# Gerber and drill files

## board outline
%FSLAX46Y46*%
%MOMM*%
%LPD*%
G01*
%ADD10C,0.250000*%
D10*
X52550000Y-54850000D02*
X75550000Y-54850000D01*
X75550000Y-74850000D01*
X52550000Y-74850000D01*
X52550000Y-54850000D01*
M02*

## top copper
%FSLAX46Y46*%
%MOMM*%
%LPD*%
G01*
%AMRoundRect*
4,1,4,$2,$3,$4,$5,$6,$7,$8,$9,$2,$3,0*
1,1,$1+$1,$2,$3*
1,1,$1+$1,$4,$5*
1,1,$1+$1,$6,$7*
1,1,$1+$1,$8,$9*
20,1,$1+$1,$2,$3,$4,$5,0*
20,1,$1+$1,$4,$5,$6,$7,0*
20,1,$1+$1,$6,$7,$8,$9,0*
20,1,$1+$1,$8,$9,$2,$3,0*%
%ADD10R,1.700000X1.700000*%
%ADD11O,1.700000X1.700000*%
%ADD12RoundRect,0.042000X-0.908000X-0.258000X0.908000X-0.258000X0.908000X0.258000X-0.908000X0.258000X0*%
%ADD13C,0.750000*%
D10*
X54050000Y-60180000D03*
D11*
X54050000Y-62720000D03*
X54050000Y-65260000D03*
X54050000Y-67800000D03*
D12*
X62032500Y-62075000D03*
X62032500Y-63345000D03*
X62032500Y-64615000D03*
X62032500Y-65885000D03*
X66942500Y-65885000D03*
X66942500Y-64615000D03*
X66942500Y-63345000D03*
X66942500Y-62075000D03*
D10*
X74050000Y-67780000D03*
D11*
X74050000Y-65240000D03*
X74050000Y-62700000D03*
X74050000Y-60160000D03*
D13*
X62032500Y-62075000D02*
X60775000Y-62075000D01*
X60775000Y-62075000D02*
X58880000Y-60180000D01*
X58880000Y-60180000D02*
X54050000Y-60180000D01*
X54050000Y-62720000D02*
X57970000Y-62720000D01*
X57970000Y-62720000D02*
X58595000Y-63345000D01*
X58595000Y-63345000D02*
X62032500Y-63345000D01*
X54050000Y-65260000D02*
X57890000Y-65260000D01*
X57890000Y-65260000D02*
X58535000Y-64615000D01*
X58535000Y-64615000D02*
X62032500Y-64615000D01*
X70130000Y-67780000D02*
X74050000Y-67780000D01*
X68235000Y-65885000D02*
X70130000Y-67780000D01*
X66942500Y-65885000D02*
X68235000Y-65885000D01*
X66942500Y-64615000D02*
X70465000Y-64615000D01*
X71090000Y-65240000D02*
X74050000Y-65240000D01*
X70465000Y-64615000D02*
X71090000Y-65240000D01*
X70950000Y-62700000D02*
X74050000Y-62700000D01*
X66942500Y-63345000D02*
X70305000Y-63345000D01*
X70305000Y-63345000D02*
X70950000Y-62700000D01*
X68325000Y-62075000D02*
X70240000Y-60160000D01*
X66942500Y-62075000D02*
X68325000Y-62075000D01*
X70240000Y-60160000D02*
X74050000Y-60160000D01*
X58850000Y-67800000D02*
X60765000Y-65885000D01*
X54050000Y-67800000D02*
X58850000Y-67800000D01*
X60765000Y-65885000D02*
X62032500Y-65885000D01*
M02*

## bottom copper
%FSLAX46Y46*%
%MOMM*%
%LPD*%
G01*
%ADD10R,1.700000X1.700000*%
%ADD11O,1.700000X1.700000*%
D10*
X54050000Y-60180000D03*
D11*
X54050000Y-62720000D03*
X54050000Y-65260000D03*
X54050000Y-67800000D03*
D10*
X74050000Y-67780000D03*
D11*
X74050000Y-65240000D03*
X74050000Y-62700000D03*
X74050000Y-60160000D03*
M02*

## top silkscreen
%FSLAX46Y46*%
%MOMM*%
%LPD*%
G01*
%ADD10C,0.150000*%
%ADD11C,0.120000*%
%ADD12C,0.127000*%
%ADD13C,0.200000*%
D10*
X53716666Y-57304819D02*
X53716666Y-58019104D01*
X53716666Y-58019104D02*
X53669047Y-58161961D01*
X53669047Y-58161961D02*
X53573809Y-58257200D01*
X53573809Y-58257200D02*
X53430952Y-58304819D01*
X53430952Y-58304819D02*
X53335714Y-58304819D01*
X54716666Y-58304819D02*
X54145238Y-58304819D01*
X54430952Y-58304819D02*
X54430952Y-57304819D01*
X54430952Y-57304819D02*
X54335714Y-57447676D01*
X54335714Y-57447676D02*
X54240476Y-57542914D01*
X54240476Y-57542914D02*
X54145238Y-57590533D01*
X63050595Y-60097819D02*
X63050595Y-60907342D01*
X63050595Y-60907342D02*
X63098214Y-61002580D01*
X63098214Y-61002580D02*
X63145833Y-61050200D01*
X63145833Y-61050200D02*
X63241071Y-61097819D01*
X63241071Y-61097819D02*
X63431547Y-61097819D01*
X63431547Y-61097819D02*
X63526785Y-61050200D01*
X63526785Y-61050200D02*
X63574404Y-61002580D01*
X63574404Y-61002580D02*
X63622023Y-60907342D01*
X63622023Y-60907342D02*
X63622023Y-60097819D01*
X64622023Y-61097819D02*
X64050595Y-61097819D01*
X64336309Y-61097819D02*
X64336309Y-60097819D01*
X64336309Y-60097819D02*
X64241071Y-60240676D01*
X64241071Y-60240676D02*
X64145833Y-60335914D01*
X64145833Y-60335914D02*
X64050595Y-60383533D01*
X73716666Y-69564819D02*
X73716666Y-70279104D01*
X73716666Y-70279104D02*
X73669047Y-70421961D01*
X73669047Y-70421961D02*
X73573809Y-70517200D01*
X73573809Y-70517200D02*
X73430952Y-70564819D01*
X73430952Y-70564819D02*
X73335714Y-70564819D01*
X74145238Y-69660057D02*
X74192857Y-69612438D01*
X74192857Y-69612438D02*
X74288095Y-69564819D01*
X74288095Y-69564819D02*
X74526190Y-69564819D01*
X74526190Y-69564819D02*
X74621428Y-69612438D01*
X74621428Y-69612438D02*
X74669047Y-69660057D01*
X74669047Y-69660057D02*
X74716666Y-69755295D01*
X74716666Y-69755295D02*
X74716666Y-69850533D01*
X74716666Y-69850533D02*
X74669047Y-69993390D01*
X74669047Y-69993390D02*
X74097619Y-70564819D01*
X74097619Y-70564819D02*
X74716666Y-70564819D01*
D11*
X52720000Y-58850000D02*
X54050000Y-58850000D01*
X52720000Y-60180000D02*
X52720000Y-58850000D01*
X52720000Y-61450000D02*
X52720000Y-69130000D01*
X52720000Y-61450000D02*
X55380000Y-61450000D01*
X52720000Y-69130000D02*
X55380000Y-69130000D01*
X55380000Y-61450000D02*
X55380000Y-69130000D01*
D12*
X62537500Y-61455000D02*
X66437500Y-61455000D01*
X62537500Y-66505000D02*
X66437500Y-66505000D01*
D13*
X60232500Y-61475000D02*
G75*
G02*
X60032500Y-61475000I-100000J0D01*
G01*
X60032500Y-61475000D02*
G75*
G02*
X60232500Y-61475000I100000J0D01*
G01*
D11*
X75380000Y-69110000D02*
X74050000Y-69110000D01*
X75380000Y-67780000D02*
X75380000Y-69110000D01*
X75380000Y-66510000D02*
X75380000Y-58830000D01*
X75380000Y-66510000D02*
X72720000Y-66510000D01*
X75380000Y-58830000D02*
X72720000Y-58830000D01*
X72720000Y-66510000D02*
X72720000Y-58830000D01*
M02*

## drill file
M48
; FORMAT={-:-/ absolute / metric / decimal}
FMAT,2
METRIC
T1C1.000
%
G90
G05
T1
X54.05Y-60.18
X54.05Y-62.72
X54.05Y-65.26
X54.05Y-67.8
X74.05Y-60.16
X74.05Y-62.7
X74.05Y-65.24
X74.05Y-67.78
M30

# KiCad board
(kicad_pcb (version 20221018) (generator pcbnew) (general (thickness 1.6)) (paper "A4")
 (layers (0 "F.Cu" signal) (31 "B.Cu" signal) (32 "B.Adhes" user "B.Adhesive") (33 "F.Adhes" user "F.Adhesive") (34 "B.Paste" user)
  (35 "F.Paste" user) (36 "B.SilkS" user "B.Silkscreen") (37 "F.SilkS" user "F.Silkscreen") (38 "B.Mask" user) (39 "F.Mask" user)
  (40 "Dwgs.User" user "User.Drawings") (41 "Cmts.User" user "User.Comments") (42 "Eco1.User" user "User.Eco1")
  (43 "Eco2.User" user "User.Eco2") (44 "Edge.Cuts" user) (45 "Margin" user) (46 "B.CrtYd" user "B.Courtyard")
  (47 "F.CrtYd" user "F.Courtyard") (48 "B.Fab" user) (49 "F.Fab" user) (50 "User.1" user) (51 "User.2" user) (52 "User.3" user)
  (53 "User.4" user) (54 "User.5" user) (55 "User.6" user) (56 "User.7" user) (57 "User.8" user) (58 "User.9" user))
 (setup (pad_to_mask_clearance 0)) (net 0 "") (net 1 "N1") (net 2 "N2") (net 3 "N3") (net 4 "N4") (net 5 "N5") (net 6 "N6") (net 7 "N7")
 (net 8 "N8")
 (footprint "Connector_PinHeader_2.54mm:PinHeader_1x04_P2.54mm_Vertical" (layer "F.Cu") (at 54.05 60.18)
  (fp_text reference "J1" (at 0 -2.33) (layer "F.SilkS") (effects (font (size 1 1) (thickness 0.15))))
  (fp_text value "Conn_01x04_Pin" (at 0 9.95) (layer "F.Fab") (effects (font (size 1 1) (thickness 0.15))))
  (fp_line (start -1.33 -1.33) (end 0 -1.33) (stroke (width 0.12) (type solid)) (layer "F.SilkS"))
  (fp_line (start -1.33 0) (end -1.33 -1.33) (stroke (width 0.12) (type solid)) (layer "F.SilkS"))
  (fp_line (start -1.33 1.27) (end -1.33 8.95) (stroke (width 0.12) (type solid)) (layer "F.SilkS"))
  (fp_line (start -1.33 1.27) (end 1.33 1.27) (stroke (width 0.12) (type solid)) (layer "F.SilkS"))
  (fp_line (start -1.33 8.95) (end 1.33 8.95) (stroke (width 0.12) (type solid)) (layer "F.SilkS"))
  (fp_line (start 1.33 1.27) (end 1.33 8.95) (stroke (width 0.12) (type solid)) (layer "F.SilkS"))
  (pad "1" thru_hole rect (at 0 0) (size 1.7 1.7) (drill 1) (layers "*.Cu" "*.Mask") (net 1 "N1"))
  (pad "2" thru_hole oval (at 0 2.54) (size 1.7 1.7) (drill 1) (layers "*.Cu" "*.Mask") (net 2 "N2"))
  (pad "3" thru_hole oval (at 0 5.08) (size 1.7 1.7) (drill 1) (layers "*.Cu" "*.Mask") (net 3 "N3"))
  (pad "4" thru_hole oval (at 0 7.62) (size 1.7 1.7) (drill 1) (layers "*.Cu" "*.Mask") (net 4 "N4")))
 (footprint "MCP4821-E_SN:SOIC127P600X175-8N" (layer "F.Cu") (at 64.4875 63.98)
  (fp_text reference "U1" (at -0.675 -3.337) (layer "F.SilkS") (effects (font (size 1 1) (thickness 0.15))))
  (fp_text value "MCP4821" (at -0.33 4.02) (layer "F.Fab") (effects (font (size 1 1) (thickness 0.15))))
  (fp_line (start -1.95 -2.525) (end 1.95 -2.525) (stroke (width 0.127) (type solid)) (layer "F.SilkS"))
  (fp_line (start -1.95 2.525) (end 1.95 2.525) (stroke (width 0.127) (type solid)) (layer "F.SilkS"))
  (fp_circle (center -4.355 -2.505) (end -4.255 -2.505) (stroke (width 0.2) (type solid)) (fill none) (layer "F.SilkS"))
  (pad "1" smd roundrect (at -2.455 -1.905) (size 1.9 0.6) (layers "F.Cu" "F.Paste" "F.Mask") (roundrect_rratio 0.07) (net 1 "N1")
   (solder_mask_margin 0.102))
  (pad "2" smd roundrect (at -2.455 -0.635) (size 1.9 0.6) (layers "F.Cu" "F.Paste" "F.Mask") (roundrect_rratio 0.07) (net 2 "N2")
   (solder_mask_margin 0.102))
  (pad "3" smd roundrect (at -2.455 0.635) (size 1.9 0.6) (layers "F.Cu" "F.Paste" "F.Mask") (roundrect_rratio 0.07) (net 3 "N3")
   (solder_mask_margin 0.102))
  (pad "4" smd roundrect (at -2.455 1.905) (size 1.9 0.6) (layers "F.Cu" "F.Paste" "F.Mask") (roundrect_rratio 0.07) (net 4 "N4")
   (solder_mask_margin 0.102))
  (pad "5" smd roundrect (at 2.455 1.905) (size 1.9 0.6) (layers "F.Cu" "F.Paste" "F.Mask") (roundrect_rratio 0.07) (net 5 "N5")
   (solder_mask_margin 0.102))
  (pad "6" smd roundrect (at 2.455 0.635) (size 1.9 0.6) (layers "F.Cu" "F.Paste" "F.Mask") (roundrect_rratio 0.07) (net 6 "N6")
   (solder_mask_margin 0.102))
  (pad "7" smd roundrect (at 2.455 -0.635) (size 1.9 0.6) (layers "F.Cu" "F.Paste" "F.Mask") (roundrect_rratio 0.07) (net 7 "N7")
   (solder_mask_margin 0.102))
  (pad "8" smd roundrect (at 2.455 -1.905) (size 1.9 0.6) (layers "F.Cu" "F.Paste" "F.Mask") (roundrect_rratio 0.07) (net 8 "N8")
   (solder_mask_margin 0.102)))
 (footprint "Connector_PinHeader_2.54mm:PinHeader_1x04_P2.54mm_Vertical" (layer "F.Cu") (at 74.05 67.78 180)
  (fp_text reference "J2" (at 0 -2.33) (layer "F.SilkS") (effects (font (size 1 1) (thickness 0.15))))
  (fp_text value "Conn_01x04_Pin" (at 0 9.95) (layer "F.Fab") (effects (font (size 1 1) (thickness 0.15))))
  (fp_line (start -1.33 -1.33) (end 0 -1.33) (stroke (width 0.12) (type solid)) (layer "F.SilkS"))
  (fp_line (start -1.33 0) (end -1.33 -1.33) (stroke (width 0.12) (type solid)) (layer "F.SilkS"))
  (fp_line (start -1.33 1.27) (end -1.33 8.95) (stroke (width 0.12) (type solid)) (layer "F.SilkS"))
  (fp_line (start -1.33 1.27) (end 1.33 1.27) (stroke (width 0.12) (type solid)) (layer "F.SilkS"))
  (fp_line (start -1.33 8.95) (end 1.33 8.95) (stroke (width 0.12) (type solid)) (layer "F.SilkS"))
  (fp_line (start 1.33 1.27) (end 1.33 8.95) (stroke (width 0.12) (type solid)) (layer "F.SilkS"))
  (pad "1" thru_hole rect (at 0 0 180) (size 1.7 1.7) (drill 1) (layers "*.Cu" "*.Mask") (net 5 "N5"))
  (pad "2" thru_hole oval (at 0 2.54 180) (size 1.7 1.7) (drill 1) (layers "*.Cu" "*.Mask") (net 6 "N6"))
  (pad "3" thru_hole oval (at 0 5.08 180) (size 1.7 1.7) (drill 1) (layers "*.Cu" "*.Mask") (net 7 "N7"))
  (pad "4" thru_hole oval (at 0 7.62 180) (size 1.7 1.7) (drill 1) (layers "*.Cu" "*.Mask") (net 8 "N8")))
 (gr_rect (start 52.55 54.85) (end 75.55 74.85) (stroke (width 0.25) (type default)) (fill none) (layer "Edge.Cuts"))
 (segment (start 62.0325 62.075) (end 60.775 62.075) (width 0.75) (layer "F.Cu") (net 1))
 (segment (start 60.775 62.075) (end 58.88 60.18) (width 0.75) (layer "F.Cu") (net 1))
 (segment (start 58.88 60.18) (end 54.05 60.18) (width 0.75) (layer "F.Cu") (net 1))
 (segment (start 54.05 62.72) (end 57.97 62.72) (width 0.75) (layer "F.Cu") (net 2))
 (segment (start 57.97 62.72) (end 58.595 63.345) (width 0.75) (layer "F.Cu") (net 2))
 (segment (start 58.595 63.345) (end 62.0325 63.345) (width 0.75) (layer "F.Cu") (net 2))
 (segment (start 54.05 65.26) (end 57.89 65.26) (width 0.75) (layer "F.Cu") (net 3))
 (segment (start 57.89 65.26) (end 58.535 64.615) (width 0.75) (layer "F.Cu") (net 3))
 (segment (start 58.535 64.615) (end 62.0325 64.615) (width 0.75) (layer "F.Cu") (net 3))
 (segment (start 70.13 67.78) (end 74.05 67.78) (width 0.75) (layer "F.Cu") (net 5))
 (segment (start 68.235 65.885) (end 70.13 67.78) (width 0.75) (layer "F.Cu") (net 5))
 (segment (start 66.9425 65.885) (end 68.235 65.885) (width 0.75) (layer "F.Cu") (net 5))
 (segment (start 66.9425 64.615) (end 70.465 64.615) (width 0.75) (layer "F.Cu") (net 6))
 (segment (start 71.09 65.24) (end 74.05 65.24) (width 0.75) (layer "F.Cu") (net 6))
 (segment (start 70.465 64.615) (end 71.09 65.24) (width 0.75) (layer "F.Cu") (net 6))
 (segment (start 70.95 62.7) (end 74.05 62.7) (width 0.75) (layer "F.Cu") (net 7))
 (segment (start 66.9425 63.345) (end 70.305 63.345) (width 0.75) (layer "F.Cu") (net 7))
 (segment (start 70.305 63.345) (end 70.95 62.7) (width 0.75) (layer "F.Cu") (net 7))
 (segment (start 68.325 62.075) (end 70.24 60.16) (width 0.75) (layer "F.Cu") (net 8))
 (segment (start 66.9425 62.075) (end 68.325 62.075) (width 0.75) (layer "F.Cu") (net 8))
 (segment (start 70.24 60.16) (end 74.05 60.16) (width 0.75) (layer "F.Cu") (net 8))
 (segment (start 58.85 67.8) (end 60.765 65.885) (width 0.75) (layer "F.Cu") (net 4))
 (segment (start 54.05 67.8) (end 58.85 67.8) (width 0.75) (layer "F.Cu") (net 4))
 (segment (start 60.765 65.885) (end 62.0325 65.885) (width 0.75) (layer "F.Cu") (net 4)))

